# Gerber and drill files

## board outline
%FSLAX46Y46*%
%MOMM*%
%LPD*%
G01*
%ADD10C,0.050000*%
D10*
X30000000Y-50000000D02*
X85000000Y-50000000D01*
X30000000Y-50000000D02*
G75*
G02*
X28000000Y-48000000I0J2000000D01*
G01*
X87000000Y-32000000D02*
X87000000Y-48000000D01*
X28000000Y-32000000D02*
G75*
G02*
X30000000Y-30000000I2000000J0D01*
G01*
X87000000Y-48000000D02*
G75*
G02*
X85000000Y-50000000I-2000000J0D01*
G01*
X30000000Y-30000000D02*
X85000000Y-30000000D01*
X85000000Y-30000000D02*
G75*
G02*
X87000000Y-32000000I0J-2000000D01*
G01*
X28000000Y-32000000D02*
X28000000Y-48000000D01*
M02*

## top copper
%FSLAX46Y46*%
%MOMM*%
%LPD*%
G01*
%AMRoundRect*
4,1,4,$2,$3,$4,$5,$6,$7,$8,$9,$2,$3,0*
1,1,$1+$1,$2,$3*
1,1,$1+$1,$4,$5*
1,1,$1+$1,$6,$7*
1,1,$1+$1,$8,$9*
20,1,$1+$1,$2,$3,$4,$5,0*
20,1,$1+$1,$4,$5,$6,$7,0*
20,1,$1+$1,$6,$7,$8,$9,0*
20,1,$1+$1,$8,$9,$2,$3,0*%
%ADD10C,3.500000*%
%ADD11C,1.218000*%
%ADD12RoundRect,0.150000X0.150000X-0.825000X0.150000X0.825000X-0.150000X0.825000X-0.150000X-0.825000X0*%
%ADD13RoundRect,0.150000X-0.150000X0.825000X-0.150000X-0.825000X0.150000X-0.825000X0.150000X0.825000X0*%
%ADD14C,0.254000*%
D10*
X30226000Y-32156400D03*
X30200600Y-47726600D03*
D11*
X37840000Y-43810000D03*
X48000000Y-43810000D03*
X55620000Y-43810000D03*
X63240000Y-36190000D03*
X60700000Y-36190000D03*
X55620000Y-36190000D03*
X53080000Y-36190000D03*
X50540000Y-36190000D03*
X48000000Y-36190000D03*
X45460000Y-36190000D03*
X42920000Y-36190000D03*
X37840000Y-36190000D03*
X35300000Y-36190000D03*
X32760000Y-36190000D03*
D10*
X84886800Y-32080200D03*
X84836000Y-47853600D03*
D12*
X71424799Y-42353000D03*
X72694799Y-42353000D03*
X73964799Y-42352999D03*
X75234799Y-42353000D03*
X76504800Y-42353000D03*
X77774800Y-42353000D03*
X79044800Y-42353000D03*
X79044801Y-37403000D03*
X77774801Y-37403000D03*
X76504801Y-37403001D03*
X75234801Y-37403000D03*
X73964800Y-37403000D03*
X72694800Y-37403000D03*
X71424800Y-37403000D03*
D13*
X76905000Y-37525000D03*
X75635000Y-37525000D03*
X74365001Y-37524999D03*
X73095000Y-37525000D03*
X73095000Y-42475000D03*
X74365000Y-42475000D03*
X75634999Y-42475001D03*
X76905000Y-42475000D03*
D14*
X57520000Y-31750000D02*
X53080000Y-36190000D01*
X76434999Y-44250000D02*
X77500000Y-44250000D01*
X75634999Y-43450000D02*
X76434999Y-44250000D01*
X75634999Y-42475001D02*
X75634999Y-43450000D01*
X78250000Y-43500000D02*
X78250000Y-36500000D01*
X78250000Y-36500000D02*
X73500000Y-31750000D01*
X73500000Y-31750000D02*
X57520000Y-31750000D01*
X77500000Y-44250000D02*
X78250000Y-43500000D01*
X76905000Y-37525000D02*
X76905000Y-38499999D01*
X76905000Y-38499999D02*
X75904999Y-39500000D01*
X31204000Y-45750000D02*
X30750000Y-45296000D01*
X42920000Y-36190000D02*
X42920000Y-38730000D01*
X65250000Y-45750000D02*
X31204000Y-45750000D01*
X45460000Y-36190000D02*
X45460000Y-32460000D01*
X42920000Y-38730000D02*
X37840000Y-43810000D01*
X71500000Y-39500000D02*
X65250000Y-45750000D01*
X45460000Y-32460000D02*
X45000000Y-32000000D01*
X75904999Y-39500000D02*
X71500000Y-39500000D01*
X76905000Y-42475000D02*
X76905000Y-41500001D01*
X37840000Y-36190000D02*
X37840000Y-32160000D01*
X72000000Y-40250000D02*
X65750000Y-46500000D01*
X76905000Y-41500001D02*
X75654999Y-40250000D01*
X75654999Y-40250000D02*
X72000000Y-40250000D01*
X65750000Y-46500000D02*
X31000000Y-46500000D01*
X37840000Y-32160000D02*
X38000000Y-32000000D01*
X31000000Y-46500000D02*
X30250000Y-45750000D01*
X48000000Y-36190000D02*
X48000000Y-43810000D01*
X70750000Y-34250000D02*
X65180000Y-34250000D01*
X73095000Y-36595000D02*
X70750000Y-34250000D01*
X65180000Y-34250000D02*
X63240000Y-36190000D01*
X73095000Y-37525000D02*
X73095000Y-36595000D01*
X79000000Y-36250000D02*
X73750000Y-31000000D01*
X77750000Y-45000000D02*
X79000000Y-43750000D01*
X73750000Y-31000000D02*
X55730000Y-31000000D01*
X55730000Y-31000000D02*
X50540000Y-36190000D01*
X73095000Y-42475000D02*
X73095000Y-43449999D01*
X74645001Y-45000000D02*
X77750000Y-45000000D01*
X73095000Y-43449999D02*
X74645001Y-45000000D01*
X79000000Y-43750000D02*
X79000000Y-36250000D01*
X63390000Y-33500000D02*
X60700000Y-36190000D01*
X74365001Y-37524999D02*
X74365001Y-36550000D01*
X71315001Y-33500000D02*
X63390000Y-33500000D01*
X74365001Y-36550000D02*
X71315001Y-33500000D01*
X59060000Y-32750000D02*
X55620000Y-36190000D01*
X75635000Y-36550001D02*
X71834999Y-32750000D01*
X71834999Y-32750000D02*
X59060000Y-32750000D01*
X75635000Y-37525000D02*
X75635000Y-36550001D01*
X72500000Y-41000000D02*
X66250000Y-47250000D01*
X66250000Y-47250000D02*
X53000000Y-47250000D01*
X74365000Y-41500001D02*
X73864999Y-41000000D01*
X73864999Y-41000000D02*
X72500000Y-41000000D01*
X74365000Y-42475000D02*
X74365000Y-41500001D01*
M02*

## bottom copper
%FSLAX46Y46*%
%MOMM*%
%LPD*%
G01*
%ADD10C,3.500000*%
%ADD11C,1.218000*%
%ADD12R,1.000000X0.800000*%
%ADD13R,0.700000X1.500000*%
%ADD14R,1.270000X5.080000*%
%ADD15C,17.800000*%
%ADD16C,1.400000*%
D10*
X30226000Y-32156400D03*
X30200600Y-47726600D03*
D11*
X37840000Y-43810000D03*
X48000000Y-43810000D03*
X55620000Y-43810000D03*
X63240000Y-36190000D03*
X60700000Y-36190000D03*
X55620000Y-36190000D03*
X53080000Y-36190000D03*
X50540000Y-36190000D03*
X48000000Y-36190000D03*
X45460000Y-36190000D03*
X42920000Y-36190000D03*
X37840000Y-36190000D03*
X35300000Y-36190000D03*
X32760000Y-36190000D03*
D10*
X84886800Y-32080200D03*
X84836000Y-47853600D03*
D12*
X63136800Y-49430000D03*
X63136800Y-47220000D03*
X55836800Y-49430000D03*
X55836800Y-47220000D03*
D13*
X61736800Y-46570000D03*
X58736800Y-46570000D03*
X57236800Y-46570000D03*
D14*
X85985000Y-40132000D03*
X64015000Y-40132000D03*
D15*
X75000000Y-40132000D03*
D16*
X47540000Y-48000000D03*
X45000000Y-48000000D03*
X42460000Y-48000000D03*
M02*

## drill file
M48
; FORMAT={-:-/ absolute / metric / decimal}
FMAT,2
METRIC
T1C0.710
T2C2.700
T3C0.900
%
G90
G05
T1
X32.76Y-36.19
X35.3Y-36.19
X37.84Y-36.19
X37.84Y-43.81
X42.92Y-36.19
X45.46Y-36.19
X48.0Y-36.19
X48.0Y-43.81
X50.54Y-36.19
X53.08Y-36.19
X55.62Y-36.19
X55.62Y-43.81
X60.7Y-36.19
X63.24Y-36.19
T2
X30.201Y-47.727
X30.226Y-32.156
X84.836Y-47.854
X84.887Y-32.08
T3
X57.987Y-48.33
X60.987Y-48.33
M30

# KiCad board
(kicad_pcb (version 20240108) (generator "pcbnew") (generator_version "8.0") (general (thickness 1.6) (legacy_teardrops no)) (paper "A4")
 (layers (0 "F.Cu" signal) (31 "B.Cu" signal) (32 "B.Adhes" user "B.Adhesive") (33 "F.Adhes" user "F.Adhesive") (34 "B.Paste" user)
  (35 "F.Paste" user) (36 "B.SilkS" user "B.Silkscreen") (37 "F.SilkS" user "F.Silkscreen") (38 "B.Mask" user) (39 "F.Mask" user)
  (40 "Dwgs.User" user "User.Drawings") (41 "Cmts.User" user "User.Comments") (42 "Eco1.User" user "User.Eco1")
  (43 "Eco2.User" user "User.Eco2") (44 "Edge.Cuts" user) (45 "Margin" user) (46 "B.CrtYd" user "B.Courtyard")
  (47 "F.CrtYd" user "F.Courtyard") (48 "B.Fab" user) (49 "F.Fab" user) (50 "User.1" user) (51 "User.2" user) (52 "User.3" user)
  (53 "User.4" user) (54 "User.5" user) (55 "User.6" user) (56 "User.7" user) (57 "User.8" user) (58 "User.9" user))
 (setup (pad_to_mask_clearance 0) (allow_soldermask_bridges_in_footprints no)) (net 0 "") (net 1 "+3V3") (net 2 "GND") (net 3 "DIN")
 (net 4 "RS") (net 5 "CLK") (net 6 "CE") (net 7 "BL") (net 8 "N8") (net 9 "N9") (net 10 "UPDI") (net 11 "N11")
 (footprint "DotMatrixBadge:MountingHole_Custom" (layer "F.Cu") (at 30.226 32.1564)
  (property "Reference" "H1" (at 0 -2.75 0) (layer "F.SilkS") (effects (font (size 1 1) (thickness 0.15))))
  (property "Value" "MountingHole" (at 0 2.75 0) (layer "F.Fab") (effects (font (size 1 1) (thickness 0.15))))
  (pad "1" thru_hole circle (at 0 0) (size 3.5 3.5) (drill 2.7) (layers "*.Cu" "*.Mask") (remove_unused_layers no)))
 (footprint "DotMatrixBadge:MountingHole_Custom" (layer "F.Cu") (at 30.2006 47.7266)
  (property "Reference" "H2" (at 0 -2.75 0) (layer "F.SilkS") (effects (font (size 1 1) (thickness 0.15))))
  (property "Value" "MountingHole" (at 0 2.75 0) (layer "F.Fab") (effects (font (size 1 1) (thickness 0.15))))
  (pad "1" thru_hole circle (at 0 0) (size 3.5 3.5) (drill 2.7) (layers "*.Cu" "*.Mask") (remove_unused_layers no)))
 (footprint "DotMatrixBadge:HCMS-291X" (layer "F.Cu") (at 48 40)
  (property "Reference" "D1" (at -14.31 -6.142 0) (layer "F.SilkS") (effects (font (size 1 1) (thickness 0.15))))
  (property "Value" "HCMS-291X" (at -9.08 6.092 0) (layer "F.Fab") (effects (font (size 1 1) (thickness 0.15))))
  (pad "3" thru_hole circle (at -10.16 3.81) (size 1.218 1.218) (drill 0.71) (layers "*.Cu" "*.Mask") (remove_unused_layers no)
   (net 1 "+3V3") (solder_mask_margin 0.102))
  (pad "7" thru_hole circle (at 0 3.81) (size 1.218 1.218) (drill 0.71) (layers "*.Cu" "*.Mask") (remove_unused_layers no) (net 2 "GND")
   (solder_mask_margin 0.102))
  (pad "10" thru_hole circle (at 7.62 3.81) (size 1.218 1.218) (drill 0.71) (layers "*.Cu" "*.Mask") (remove_unused_layers no)
   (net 1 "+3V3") (solder_mask_margin 0.102))
  (pad "14" thru_hole circle (at 15.24 -3.81) (size 1.218 1.218) (drill 0.71) (layers "*.Cu" "*.Mask") (remove_unused_layers no)
   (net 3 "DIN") (solder_mask_margin 0.102))
  (pad "15" thru_hole circle (at 12.7 -3.81) (size 1.218 1.218) (drill 0.71) (layers "*.Cu" "*.Mask") (remove_unused_layers no) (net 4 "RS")
   (solder_mask_margin 0.102))
  (pad "17" thru_hole circle (at 7.62 -3.81) (size 1.218 1.218) (drill 0.71) (layers "*.Cu" "*.Mask") (remove_unused_layers no)
   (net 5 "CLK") (solder_mask_margin 0.102))
  (pad "18" thru_hole circle (at 5.08 -3.81) (size 1.218 1.218) (drill 0.71) (layers "*.Cu" "*.Mask") (remove_unused_layers no) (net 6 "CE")
   (solder_mask_margin 0.102))
  (pad "19" thru_hole circle (at 2.54 -3.81) (size 1.218 1.218) (drill 0.71) (layers "*.Cu" "*.Mask") (remove_unused_layers no) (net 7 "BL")
   (solder_mask_margin 0.102))
  (pad "20" thru_hole circle (at 0 -3.81) (size 1.218 1.218) (drill 0.71) (layers "*.Cu" "*.Mask") (remove_unused_layers no) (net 2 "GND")
   (solder_mask_margin 0.102))
  (pad "21" thru_hole circle (at -2.54 -3.81) (size 1.218 1.218) (drill 0.71) (layers "*.Cu" "*.Mask") (remove_unused_layers no)
   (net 1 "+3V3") (solder_mask_margin 0.102))
  (pad "22" thru_hole circle (at -5.08 -3.81) (size 1.218 1.218) (drill 0.71) (layers "*.Cu" "*.Mask") (remove_unused_layers no)
   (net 1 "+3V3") (solder_mask_margin 0.102))
  (pad "24" thru_hole circle (at -10.16 -3.81) (size 1.218 1.218) (drill 0.71) (layers "*.Cu" "*.Mask") (remove_unused_layers no)
   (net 2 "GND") (solder_mask_margin 0.102))
  (pad "25" thru_hole circle (at -12.7 -3.81) (size 1.218 1.218) (drill 0.71) (layers "*.Cu" "*.Mask") (remove_unused_layers no)
   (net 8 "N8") (solder_mask_margin 0.102))
  (pad "26" thru_hole circle (at -15.24 -3.81) (size 1.218 1.218) (drill 0.71) (layers "*.Cu" "*.Mask") (remove_unused_layers no)
   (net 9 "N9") (solder_mask_margin 0.102)))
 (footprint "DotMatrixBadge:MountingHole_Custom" (layer "F.Cu") (at 84.8868 32.0802)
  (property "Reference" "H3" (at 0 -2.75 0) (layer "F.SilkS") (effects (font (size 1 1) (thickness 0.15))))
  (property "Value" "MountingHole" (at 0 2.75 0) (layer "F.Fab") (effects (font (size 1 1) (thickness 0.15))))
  (pad "1" thru_hole circle (at 0 0) (size 3.5 3.5) (drill 2.7) (layers "*.Cu" "*.Mask") (remove_unused_layers no)))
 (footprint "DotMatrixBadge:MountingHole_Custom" (layer "F.Cu") (at 84.836 47.8536)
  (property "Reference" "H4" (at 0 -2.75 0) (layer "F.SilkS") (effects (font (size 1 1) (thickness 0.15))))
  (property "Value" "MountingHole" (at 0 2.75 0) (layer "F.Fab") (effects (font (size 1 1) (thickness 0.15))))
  (pad "1" thru_hole circle (at 0 0) (size 3.5 3.5) (drill 2.7) (layers "*.Cu" "*.Mask") (remove_unused_layers no)))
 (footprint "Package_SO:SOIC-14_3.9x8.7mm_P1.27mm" (layer "F.Cu") (at 75.2348 39.878 90)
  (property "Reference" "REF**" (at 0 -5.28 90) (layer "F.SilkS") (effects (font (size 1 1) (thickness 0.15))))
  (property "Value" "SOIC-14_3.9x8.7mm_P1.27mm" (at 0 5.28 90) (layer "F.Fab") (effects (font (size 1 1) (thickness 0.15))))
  (pad "1" smd roundrect (at -2.475 -3.810001 90) (size 1.95 0.6) (layers "F.Cu" "F.Paste" "F.Mask") (roundrect_rratio 0.25))
  (pad "2" smd roundrect (at -2.475 -2.540001 90) (size 1.95 0.6) (layers "F.Cu" "F.Paste" "F.Mask") (roundrect_rratio 0.25))
  (pad "3" smd roundrect (at -2.474999 -1.270001 90) (size 1.95 0.6) (layers "F.Cu" "F.Paste" "F.Mask") (roundrect_rratio 0.25))
  (pad "4" smd roundrect (at -2.475 -0.000001 90) (size 1.95 0.6) (layers "F.Cu" "F.Paste" "F.Mask") (roundrect_rratio 0.25))
  (pad "5" smd roundrect (at -2.475 1.27 90) (size 1.95 0.6) (layers "F.Cu" "F.Paste" "F.Mask") (roundrect_rratio 0.25))
  (pad "6" smd roundrect (at -2.475 2.54 90) (size 1.95 0.6) (layers "F.Cu" "F.Paste" "F.Mask") (roundrect_rratio 0.25))
  (pad "7" smd roundrect (at -2.475 3.81 90) (size 1.95 0.6) (layers "F.Cu" "F.Paste" "F.Mask") (roundrect_rratio 0.25))
  (pad "8" smd roundrect (at 2.475 3.810001 90) (size 1.95 0.6) (layers "F.Cu" "F.Paste" "F.Mask") (roundrect_rratio 0.25))
  (pad "9" smd roundrect (at 2.475 2.540001 90) (size 1.95 0.6) (layers "F.Cu" "F.Paste" "F.Mask") (roundrect_rratio 0.25))
  (pad "10" smd roundrect (at 2.474999 1.270001 90) (size 1.95 0.6) (layers "F.Cu" "F.Paste" "F.Mask") (roundrect_rratio 0.25))
  (pad "11" smd roundrect (at 2.475 0.000001 90) (size 1.95 0.6) (layers "F.Cu" "F.Paste" "F.Mask") (roundrect_rratio 0.25))
  (pad "12" smd roundrect (at 2.475 -1.27 90) (size 1.95 0.6) (layers "F.Cu" "F.Paste" "F.Mask") (roundrect_rratio 0.25))
  (pad "13" smd roundrect (at 2.475 -2.54 90) (size 1.95 0.6) (layers "F.Cu" "F.Paste" "F.Mask") (roundrect_rratio 0.25))
  (pad "14" smd roundrect (at 2.475 -3.81 90) (size 1.95 0.6) (layers "F.Cu" "F.Paste" "F.Mask") (roundrect_rratio 0.25)))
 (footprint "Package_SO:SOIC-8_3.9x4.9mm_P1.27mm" (layer "F.Cu") (at 75 40 -90)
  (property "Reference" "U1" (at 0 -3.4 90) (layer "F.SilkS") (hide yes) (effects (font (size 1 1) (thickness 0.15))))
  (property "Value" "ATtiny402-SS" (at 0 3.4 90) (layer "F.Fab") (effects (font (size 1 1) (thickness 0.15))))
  (pad "1" smd roundrect (at -2.475 -1.905 270) (size 1.95 0.6) (layers "F.Cu" "F.Paste" "F.Mask") (roundrect_rratio 0.25) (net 1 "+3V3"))
  (pad "2" smd roundrect (at -2.475 -0.635 270) (size 1.95 0.6) (layers "F.Cu" "F.Paste" "F.Mask") (roundrect_rratio 0.25) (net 5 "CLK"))
  (pad "3" smd roundrect (at -2.475001 0.634999 270) (size 1.95 0.6) (layers "F.Cu" "F.Paste" "F.Mask") (roundrect_rratio 0.25) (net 4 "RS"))
  (pad "4" smd roundrect (at -2.475 1.905 270) (size 1.95 0.6) (layers "F.Cu" "F.Paste" "F.Mask") (roundrect_rratio 0.25) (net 3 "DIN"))
  (pad "5" smd roundrect (at 2.475 1.905 270) (size 1.95 0.6) (layers "F.Cu" "F.Paste" "F.Mask") (roundrect_rratio 0.25) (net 7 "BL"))
  (pad "6" smd roundrect (at 2.475 0.635 270) (size 1.95 0.6) (layers "F.Cu" "F.Paste" "F.Mask") (roundrect_rratio 0.25) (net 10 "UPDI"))
  (pad "7" smd roundrect (at 2.475001 -0.634999 270) (size 1.95 0.6) (layers "F.Cu" "F.Paste" "F.Mask") (roundrect_rratio 0.25) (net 6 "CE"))
  (pad "8" smd roundrect (at 2.475 -1.905 270) (size 1.95 0.6) (layers "F.Cu" "F.Paste" "F.Mask") (roundrect_rratio 0.25) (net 2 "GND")))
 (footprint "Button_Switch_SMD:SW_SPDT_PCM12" (layer "B.Cu") (at 59.4868 48 180)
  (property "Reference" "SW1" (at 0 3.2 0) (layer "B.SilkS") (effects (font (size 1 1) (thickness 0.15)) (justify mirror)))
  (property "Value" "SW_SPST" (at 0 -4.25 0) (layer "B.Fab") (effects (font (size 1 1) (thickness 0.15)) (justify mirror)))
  (pad "" smd rect (at -3.65 -1.43 180) (size 1 0.8) (layers "B.Cu" "B.Paste" "B.Mask"))
  (pad "" smd rect (at -3.65 0.78 180) (size 1 0.8) (layers "B.Cu" "B.Paste" "B.Mask"))
  (pad "" np_thru_hole circle (at -1.5 -0.33 180) (size 0.9 0.9) (drill 0.9) (layers "*.Cu" "*.Mask"))
  (pad "" np_thru_hole circle (at 1.5 -0.33 180) (size 0.9 0.9) (drill 0.9) (layers "*.Cu" "*.Mask"))
  (pad "" smd rect (at 3.65 -1.43 180) (size 1 0.8) (layers "B.Cu" "B.Paste" "B.Mask"))
  (pad "" smd rect (at 3.65 0.78 180) (size 1 0.8) (layers "B.Cu" "B.Paste" "B.Mask"))
  (pad "1" smd rect (at -2.25 1.43 180) (size 0.7 1.5) (layers "B.Cu" "B.Paste" "B.Mask") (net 1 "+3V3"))
  (pad "2" smd rect (at 0.75 1.43 180) (size 0.7 1.5) (layers "B.Cu" "B.Paste" "B.Mask") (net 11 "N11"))
  (pad "3" smd rect (at 2.25 1.43 180) (size 0.7 1.5) (layers "B.Cu" "B.Paste" "B.Mask")))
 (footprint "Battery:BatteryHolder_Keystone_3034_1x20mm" (layer "B.Cu") (at 75 40.132 180)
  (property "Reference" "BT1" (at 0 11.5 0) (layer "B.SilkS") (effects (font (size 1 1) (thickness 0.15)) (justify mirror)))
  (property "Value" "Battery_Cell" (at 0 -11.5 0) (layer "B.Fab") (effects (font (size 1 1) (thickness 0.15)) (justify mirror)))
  (pad "1" smd rect (at -10.985 0 180) (size 1.27 5.08) (layers "B.Cu" "B.Paste" "B.Mask") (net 11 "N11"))
  (pad "1" smd rect (at 10.985 0 180) (size 1.27 5.08) (layers "B.Cu" "B.Paste" "B.Mask") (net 11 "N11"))
  (pad "2" smd circle (at 0 0 180) (size 17.8 17.8) (layers "B.Cu" "B.Mask") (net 2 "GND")))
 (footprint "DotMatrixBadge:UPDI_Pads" (layer "B.Cu") (at 47.54 48 180)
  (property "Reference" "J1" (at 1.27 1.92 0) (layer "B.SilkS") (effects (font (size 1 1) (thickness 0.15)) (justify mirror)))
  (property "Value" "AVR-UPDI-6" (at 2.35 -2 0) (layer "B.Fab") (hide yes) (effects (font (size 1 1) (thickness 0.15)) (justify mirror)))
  (pad "1" smd circle (at 0 0 180) (size 1.4 1.4) (layers "B.Cu" "B.Mask") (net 10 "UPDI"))
  (pad "2" smd circle (at 2.54 0 180) (size 1.4 1.4) (layers "B.Cu" "B.Mask") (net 1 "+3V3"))
  (pad "6" smd circle (at 5.08 0 180) (size 1.4 1.4) (layers "B.Cu" "B.Mask") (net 2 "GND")))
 (gr_line (start 30 50) (end 85 50) (stroke (width 0.05) (type default)) (layer "Edge.Cuts"))
 (gr_arc (start 30 50) (mid 28.585786 49.414214) (end 28 48) (stroke (width 0.05) (type default)) (layer "Edge.Cuts"))
 (gr_line (start 87 32) (end 87 48) (stroke (width 0.05) (type default)) (layer "Edge.Cuts"))
 (gr_arc (start 28 32) (mid 28.585786 30.585786) (end 30 30) (stroke (width 0.05) (type default)) (layer "Edge.Cuts"))
 (gr_arc (start 87 48) (mid 86.414214 49.414214) (end 85 50) (stroke (width 0.05) (type default)) (layer "Edge.Cuts"))
 (gr_line (start 30 30) (end 85 30) (stroke (width 0.05) (type default)) (layer "Edge.Cuts"))
 (gr_arc (start 85 30) (mid 86.414214 30.585786) (end 87 32) (stroke (width 0.05) (type default)) (layer "Edge.Cuts"))
 (gr_line (start 28 32) (end 28 48) (stroke (width 0.05) (type default)) (layer "Edge.Cuts"))
 (segment (start 57.52 31.75) (end 53.08 36.19) (width 0.254) (layer "F.Cu") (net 6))
 (segment (start 76.434999 44.25) (end 77.5 44.25) (width 0.254) (layer "F.Cu") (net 6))
 (segment (start 75.634999 43.45) (end 76.434999 44.25) (width 0.254) (layer "F.Cu") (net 6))
 (segment (start 75.634999 42.475001) (end 75.634999 43.45) (width 0.254) (layer "F.Cu") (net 6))
 (segment (start 78.25 43.5) (end 78.25 36.5) (width 0.254) (layer "F.Cu") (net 6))
 (segment (start 78.25 36.5) (end 73.5 31.75) (width 0.254) (layer "F.Cu") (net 6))
 (segment (start 73.5 31.75) (end 57.52 31.75) (width 0.254) (layer "F.Cu") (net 6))
 (segment (start 77.5 44.25) (end 78.25 43.5) (width 0.254) (layer "F.Cu") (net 6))
 (segment (start 76.905 37.525) (end 76.905 38.499999) (width 0.254) (layer "F.Cu") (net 1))
 (segment (start 76.905 38.499999) (end 75.904999 39.5) (width 0.254) (layer "F.Cu") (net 1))
 (segment (start 31.204 45.75) (end 30.75 45.296) (width 0.254) (layer "F.Cu") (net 1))
 (segment (start 42.92 36.19) (end 42.92 38.73) (width 0.254) (layer "F.Cu") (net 1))
 (segment (start 65.25 45.75) (end 31.204 45.75) (width 0.254) (layer "F.Cu") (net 1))
 (segment (start 45.46 36.19) (end 45.46 32.46) (width 0.254) (layer "F.Cu") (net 1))
 (segment (start 42.92 38.73) (end 37.84 43.81) (width 0.254) (layer "F.Cu") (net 1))
 (segment (start 71.5 39.5) (end 65.25 45.75) (width 0.254) (layer "F.Cu") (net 1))
 (segment (start 45.46 32.46) (end 45 32) (width 0.254) (layer "F.Cu") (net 1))
 (segment (start 75.904999 39.5) (end 71.5 39.5) (width 0.254) (layer "F.Cu") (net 1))
 (segment (start 76.905 42.475) (end 76.905 41.500001) (width 0.254) (layer "F.Cu") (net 2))
 (segment (start 37.84 36.19) (end 37.84 32.16) (width 0.254) (layer "F.Cu") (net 2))
 (segment (start 72 40.25) (end 65.75 46.5) (width 0.254) (layer "F.Cu") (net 2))
 (segment (start 76.905 41.500001) (end 75.654999 40.25) (width 0.254) (layer "F.Cu") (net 2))
 (segment (start 75.654999 40.25) (end 72 40.25) (width 0.254) (layer "F.Cu") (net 2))
 (segment (start 65.75 46.5) (end 31 46.5) (width 0.254) (layer "F.Cu") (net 2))
 (segment (start 37.84 32.16) (end 38 32) (width 0.254) (layer "F.Cu") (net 2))
 (segment (start 31 46.5) (end 30.25 45.75) (width 0.254) (layer "F.Cu") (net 2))
 (segment (start 48 36.19) (end 48 43.81) (width 0.254) (layer "F.Cu") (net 2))
 (segment (start 70.75 34.25) (end 65.18 34.25) (width 0.254) (layer "F.Cu") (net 3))
 (segment (start 73.095 36.595) (end 70.75 34.25) (width 0.254) (layer "F.Cu") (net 3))
 (segment (start 65.18 34.25) (end 63.24 36.19) (width 0.254) (layer "F.Cu") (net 3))
 (segment (start 73.095 37.525) (end 73.095 36.595) (width 0.254) (layer "F.Cu") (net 3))
 (segment (start 79 36.25) (end 73.75 31) (width 0.254) (layer "F.Cu") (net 7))
 (segment (start 77.75 45) (end 79 43.75) (width 0.254) (layer "F.Cu") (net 7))
 (segment (start 73.75 31) (end 55.73 31) (width 0.254) (layer "F.Cu") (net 7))
 (segment (start 55.73 31) (end 50.54 36.19) (width 0.254) (layer "F.Cu") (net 7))
 (segment (start 73.095 42.475) (end 73.095 43.449999) (width 0.254) (layer "F.Cu") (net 7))
 (segment (start 74.645001 45) (end 77.75 45) (width 0.254) (layer "F.Cu") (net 7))
 (segment (start 73.095 43.449999) (end 74.645001 45) (width 0.254) (layer "F.Cu") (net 7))
 (segment (start 79 43.75) (end 79 36.25) (width 0.254) (layer "F.Cu") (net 7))
 (segment (start 63.39 33.5) (end 60.7 36.19) (width 0.254) (layer "F.Cu") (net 4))
 (segment (start 74.365001 37.524999) (end 74.365001 36.55) (width 0.254) (layer "F.Cu") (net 4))
 (segment (start 71.315001 33.5) (end 63.39 33.5) (width 0.254) (layer "F.Cu") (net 4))
 (segment (start 74.365001 36.55) (end 71.315001 33.5) (width 0.254) (layer "F.Cu") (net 4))
 (segment (start 59.06 32.75) (end 55.62 36.19) (width 0.254) (layer "F.Cu") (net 5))
 (segment (start 75.635 36.550001) (end 71.834999 32.75) (width 0.254) (layer "F.Cu") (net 5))
 (segment (start 71.834999 32.75) (end 59.06 32.75) (width 0.254) (layer "F.Cu") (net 5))
 (segment (start 75.635 37.525) (end 75.635 36.550001) (width 0.254) (layer "F.Cu") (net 5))
 (segment (start 72.5 41) (end 66.25 47.25) (width 0.254) (layer "F.Cu") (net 10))
 (segment (start 66.25 47.25) (end 53 47.25) (width 0.254) (layer "F.Cu") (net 10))
 (segment (start 74.365 41.500001) (end 73.864999 41) (width 0.254) (layer "F.Cu") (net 10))
 (segment (start 73.864999 41) (end 72.5 41) (width 0.254) (layer "F.Cu") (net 10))
 (segment (start 74.365 42.475) (end 74.365 41.500001) (width 0.254) (layer "F.Cu") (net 10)))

